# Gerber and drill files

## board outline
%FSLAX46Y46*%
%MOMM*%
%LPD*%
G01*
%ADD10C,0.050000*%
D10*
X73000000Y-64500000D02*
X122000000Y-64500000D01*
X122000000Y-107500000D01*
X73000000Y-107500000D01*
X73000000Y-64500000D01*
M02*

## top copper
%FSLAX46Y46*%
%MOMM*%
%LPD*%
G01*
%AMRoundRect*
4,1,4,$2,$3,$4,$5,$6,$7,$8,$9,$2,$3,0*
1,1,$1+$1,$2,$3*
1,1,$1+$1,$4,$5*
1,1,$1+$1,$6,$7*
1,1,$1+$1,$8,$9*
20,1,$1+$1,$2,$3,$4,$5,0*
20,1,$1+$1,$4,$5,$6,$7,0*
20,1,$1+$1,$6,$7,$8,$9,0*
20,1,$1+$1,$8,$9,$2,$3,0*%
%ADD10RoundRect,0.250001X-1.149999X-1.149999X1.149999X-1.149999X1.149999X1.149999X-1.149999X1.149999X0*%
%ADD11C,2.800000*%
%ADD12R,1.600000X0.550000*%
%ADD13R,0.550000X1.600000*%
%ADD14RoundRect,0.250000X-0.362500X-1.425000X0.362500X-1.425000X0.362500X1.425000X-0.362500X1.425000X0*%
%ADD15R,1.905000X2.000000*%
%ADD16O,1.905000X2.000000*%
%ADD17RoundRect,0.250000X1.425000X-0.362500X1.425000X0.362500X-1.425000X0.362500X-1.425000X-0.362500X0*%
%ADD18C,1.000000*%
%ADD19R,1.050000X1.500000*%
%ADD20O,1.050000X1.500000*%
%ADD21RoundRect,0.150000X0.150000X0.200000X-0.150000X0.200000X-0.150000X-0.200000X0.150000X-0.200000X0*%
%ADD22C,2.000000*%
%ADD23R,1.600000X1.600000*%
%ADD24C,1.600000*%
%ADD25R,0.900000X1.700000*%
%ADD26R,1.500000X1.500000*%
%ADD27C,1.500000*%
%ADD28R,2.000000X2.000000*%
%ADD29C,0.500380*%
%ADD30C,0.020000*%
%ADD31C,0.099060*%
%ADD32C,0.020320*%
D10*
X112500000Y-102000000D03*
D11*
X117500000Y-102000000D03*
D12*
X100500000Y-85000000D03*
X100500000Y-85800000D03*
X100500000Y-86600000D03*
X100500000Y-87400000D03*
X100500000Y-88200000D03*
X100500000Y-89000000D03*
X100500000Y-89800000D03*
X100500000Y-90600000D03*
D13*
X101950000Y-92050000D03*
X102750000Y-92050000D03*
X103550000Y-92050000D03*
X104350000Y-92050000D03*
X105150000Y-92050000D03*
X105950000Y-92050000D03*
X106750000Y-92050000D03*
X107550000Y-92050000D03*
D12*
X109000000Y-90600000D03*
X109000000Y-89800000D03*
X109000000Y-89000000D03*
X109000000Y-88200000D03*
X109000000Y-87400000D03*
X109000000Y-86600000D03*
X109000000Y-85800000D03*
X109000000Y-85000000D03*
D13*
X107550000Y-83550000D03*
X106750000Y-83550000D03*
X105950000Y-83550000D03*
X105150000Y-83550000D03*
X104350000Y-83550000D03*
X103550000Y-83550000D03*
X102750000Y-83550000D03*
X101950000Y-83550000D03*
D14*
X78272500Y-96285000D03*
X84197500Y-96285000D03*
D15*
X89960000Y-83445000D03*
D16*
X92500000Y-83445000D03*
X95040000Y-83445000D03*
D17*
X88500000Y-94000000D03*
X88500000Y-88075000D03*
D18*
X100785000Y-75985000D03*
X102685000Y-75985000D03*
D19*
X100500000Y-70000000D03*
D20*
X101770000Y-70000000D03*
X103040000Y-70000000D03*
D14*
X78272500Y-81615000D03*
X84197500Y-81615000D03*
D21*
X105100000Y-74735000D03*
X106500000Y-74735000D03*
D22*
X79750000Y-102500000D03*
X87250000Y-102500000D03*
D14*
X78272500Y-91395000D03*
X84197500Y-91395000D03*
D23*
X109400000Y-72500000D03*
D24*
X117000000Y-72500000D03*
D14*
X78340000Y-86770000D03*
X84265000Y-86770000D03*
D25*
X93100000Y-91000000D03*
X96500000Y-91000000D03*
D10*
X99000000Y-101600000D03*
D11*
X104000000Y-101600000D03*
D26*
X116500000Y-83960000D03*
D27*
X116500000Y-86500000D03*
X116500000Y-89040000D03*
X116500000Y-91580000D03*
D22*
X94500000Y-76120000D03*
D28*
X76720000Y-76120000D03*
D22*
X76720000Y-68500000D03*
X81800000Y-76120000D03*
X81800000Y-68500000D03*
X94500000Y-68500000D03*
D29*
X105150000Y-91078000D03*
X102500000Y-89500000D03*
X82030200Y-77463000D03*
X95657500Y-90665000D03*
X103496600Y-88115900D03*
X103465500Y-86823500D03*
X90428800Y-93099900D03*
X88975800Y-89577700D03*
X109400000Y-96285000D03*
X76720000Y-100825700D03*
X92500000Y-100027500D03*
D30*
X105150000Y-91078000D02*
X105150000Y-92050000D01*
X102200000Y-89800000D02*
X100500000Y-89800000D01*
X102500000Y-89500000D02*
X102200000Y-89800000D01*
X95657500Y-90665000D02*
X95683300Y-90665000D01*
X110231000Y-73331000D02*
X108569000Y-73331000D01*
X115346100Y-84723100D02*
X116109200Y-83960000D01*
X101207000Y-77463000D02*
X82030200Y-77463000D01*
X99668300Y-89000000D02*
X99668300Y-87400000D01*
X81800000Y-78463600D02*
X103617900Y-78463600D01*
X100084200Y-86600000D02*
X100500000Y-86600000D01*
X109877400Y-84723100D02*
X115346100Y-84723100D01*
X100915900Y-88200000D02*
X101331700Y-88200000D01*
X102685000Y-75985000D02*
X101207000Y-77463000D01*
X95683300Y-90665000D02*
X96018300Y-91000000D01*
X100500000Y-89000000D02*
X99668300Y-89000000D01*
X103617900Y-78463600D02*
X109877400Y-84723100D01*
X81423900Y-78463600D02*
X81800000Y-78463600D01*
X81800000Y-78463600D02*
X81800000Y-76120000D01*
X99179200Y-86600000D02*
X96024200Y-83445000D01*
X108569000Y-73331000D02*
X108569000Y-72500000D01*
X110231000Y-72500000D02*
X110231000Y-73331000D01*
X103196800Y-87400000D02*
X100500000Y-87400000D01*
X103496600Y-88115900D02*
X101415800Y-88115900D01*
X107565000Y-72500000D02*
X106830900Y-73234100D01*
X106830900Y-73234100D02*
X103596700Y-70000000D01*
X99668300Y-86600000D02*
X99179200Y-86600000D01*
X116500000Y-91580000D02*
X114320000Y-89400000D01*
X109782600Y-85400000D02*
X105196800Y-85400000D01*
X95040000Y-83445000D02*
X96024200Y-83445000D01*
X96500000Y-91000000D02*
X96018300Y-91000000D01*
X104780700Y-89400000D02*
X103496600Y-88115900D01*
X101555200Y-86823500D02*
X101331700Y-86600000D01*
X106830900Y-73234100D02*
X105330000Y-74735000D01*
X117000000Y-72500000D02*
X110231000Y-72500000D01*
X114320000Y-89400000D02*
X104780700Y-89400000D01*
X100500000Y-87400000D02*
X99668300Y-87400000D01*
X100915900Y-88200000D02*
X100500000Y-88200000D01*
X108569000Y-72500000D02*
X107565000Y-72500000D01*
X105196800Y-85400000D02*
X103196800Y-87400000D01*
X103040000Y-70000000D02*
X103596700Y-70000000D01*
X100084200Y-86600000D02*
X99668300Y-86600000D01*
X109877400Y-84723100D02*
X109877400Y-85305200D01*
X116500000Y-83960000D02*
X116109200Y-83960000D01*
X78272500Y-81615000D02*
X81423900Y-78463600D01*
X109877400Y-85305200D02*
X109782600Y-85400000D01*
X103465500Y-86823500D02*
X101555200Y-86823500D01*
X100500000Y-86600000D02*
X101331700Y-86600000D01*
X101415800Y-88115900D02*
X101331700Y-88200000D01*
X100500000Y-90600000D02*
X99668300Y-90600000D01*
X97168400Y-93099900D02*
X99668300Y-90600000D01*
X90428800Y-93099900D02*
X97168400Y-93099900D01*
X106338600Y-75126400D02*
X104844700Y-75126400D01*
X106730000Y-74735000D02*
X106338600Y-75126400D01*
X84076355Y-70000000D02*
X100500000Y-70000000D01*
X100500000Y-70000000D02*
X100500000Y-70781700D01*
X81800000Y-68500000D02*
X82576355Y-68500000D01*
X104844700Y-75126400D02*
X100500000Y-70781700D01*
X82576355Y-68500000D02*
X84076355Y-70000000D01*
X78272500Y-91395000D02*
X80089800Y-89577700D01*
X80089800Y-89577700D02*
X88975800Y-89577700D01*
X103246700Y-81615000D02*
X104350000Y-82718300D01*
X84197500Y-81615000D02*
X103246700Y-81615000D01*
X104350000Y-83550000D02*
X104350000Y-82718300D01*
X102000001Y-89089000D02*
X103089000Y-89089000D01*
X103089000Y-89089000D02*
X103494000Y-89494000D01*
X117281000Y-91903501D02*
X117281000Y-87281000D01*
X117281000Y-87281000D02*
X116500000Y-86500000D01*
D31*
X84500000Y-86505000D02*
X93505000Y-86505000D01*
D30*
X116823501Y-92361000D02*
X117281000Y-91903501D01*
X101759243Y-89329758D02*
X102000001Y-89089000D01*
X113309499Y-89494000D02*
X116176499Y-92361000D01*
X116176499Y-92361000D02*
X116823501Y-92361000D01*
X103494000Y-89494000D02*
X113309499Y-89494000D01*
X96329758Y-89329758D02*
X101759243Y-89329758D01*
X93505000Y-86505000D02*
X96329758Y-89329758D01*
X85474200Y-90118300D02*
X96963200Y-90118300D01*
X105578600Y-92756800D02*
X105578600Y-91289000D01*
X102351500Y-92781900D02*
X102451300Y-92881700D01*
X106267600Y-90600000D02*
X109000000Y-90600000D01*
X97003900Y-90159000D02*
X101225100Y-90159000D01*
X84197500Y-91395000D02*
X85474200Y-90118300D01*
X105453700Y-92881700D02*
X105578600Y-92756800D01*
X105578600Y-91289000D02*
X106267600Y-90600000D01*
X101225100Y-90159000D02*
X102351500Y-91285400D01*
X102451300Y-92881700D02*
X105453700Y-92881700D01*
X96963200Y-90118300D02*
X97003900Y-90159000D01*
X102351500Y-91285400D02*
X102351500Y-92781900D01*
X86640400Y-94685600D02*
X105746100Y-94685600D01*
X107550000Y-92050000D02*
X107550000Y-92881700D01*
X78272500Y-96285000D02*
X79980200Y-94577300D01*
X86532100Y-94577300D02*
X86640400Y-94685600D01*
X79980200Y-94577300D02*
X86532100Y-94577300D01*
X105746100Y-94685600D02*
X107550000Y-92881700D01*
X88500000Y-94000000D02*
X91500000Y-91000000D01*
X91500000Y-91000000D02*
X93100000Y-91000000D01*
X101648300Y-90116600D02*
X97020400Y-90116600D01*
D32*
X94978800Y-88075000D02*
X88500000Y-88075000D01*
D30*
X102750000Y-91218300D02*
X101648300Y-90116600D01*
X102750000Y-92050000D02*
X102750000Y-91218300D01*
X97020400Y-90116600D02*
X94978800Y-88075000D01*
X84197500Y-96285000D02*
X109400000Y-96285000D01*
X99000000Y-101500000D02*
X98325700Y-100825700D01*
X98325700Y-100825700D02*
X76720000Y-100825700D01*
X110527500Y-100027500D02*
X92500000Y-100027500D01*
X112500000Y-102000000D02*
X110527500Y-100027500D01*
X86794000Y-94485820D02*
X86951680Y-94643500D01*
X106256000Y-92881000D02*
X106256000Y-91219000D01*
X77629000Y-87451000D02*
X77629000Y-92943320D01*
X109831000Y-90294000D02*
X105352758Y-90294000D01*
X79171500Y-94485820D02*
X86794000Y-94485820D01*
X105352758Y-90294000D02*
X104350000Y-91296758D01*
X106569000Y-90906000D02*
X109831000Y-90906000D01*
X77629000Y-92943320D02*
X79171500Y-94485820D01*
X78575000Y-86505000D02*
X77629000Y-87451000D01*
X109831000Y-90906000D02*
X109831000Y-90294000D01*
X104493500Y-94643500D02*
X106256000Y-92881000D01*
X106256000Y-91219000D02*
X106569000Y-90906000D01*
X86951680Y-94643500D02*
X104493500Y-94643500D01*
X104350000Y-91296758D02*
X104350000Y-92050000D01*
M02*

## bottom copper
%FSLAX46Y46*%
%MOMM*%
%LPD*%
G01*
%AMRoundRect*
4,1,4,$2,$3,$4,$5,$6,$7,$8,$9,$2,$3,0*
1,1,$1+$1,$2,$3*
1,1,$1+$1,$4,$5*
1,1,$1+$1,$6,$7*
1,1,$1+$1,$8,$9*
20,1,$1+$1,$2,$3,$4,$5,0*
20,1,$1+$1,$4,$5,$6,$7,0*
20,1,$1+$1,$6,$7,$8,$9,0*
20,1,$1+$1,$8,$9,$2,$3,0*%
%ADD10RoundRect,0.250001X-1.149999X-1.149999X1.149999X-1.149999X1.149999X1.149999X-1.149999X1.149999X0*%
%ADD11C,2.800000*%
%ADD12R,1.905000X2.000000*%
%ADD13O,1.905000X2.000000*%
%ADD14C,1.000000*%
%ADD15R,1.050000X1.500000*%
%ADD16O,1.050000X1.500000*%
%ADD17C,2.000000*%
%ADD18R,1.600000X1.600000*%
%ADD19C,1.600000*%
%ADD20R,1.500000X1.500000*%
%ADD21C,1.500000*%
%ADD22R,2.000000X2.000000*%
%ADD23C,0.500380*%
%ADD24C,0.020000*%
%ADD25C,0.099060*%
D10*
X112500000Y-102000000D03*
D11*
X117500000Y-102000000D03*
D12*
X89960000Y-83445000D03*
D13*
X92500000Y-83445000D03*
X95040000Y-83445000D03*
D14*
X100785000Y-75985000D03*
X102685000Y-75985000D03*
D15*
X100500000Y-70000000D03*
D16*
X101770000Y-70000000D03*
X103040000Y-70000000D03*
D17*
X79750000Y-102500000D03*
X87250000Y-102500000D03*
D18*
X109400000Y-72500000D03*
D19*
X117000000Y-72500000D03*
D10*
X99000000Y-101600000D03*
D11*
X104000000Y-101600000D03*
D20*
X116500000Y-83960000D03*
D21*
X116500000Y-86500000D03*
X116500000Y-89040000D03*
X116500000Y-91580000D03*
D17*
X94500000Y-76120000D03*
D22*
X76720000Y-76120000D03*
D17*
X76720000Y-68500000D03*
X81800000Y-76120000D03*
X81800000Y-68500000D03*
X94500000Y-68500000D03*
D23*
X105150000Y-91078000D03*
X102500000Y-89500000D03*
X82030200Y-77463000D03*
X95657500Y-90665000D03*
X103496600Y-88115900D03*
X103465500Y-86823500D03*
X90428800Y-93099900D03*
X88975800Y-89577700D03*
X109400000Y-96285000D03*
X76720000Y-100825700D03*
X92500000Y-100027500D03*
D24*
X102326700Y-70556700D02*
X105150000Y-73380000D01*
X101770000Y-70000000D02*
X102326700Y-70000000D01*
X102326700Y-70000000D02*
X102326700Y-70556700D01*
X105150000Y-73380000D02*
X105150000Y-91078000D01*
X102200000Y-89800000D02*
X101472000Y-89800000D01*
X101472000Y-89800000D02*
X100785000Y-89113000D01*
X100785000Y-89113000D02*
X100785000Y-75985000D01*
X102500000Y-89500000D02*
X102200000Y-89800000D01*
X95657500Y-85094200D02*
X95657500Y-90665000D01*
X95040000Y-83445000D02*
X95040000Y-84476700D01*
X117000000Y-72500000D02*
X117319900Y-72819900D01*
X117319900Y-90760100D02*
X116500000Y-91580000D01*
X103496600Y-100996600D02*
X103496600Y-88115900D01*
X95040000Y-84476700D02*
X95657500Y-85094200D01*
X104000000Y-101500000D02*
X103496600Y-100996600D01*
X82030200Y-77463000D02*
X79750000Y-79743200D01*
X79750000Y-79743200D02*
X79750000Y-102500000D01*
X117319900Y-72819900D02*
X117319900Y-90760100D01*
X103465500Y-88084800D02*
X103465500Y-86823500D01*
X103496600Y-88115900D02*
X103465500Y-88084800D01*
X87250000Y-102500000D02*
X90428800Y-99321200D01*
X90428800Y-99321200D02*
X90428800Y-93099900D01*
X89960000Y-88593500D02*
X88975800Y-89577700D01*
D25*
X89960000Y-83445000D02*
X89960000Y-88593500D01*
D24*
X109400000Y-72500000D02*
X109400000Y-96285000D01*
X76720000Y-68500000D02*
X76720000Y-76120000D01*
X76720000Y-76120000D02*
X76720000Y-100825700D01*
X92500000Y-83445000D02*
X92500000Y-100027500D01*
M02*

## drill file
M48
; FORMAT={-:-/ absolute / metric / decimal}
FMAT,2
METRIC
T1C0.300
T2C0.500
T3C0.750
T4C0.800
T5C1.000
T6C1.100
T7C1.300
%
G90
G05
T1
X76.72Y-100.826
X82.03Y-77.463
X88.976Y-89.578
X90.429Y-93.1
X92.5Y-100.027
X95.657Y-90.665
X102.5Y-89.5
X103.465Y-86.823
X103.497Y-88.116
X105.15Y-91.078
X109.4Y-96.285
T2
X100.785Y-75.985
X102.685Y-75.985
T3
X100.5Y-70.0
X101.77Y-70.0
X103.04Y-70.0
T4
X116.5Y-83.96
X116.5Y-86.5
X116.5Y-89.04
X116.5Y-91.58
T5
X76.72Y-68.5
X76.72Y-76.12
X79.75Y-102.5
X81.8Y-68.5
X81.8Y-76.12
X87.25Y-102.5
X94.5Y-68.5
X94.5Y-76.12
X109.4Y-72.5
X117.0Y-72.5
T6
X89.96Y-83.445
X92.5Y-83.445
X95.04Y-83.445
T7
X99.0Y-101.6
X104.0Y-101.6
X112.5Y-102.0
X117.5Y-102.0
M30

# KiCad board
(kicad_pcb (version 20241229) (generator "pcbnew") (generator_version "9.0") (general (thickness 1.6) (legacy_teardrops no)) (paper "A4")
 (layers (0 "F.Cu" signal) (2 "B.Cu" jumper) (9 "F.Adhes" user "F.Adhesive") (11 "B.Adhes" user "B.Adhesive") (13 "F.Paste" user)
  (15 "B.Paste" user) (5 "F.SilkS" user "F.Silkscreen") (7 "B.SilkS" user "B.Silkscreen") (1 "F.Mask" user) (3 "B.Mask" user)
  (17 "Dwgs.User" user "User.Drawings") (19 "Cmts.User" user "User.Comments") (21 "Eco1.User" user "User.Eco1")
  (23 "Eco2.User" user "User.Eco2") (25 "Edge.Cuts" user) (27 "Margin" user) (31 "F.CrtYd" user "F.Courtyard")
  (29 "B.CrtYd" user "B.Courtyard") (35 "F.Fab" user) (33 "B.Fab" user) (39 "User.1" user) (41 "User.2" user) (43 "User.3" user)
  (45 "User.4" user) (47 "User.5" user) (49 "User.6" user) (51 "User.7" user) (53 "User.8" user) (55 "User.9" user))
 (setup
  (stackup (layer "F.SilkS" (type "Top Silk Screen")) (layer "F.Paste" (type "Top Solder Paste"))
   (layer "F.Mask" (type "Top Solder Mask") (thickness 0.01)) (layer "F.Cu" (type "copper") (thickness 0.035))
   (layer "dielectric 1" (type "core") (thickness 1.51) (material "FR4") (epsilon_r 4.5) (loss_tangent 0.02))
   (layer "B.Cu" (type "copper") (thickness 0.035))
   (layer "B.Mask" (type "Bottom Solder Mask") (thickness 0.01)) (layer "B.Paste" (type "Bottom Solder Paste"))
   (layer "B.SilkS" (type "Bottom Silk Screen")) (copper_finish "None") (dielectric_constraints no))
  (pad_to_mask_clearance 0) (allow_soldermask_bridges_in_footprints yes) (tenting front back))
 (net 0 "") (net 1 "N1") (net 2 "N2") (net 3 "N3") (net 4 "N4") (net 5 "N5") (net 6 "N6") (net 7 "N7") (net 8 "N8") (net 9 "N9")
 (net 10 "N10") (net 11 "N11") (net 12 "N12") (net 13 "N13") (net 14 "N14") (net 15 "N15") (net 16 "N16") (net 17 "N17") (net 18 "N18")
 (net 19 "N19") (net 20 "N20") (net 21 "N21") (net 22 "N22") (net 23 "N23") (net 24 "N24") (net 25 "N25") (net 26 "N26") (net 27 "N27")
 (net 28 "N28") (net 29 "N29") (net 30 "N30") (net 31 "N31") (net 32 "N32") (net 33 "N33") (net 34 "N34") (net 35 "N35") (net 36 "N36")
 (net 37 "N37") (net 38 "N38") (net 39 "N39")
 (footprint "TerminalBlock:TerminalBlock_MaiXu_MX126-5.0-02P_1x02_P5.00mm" (layer "F.Cu") (at 112.5 102)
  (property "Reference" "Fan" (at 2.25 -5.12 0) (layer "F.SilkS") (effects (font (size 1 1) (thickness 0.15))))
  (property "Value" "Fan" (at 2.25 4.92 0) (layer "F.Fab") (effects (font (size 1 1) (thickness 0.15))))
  (pad "1" thru_hole roundrect (at 0 0) (size 2.8 2.8) (drill 1.3) (layers "*.Cu" "*.Mask") (remove_unused_layers no)
   (roundrect_rratio 0.089286) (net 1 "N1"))
  (pad "2" thru_hole circle (at 5 0) (size 2.8 2.8) (drill 1.3) (layers "*.Cu" "*.Mask") (remove_unused_layers no) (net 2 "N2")))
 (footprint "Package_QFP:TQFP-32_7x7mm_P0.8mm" (layer "F.Cu") (at 104.75 87.8)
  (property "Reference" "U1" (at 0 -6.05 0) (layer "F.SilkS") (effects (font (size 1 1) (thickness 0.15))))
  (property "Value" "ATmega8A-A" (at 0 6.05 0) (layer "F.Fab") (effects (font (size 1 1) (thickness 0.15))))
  (pad "1" smd rect (at -4.25 -2.8) (size 1.6 0.55) (layers "F.Cu" "F.Mask" "F.Paste") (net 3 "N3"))
  (pad "2" smd rect (at -4.25 -2) (size 1.6 0.55) (layers "F.Cu" "F.Mask" "F.Paste") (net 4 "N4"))
  (pad "3" smd rect (at -4.25 -1.2) (size 1.6 0.55) (layers "F.Cu" "F.Mask" "F.Paste") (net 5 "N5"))
  (pad "4" smd rect (at -4.25 -0.4) (size 1.6 0.55) (layers "F.Cu" "F.Mask" "F.Paste") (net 5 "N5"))
  (pad "5" smd rect (at -4.25 0.4) (size 1.6 0.55) (layers "F.Cu" "F.Mask" "F.Paste") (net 5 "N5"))
  (pad "6" smd rect (at -4.25 1.2) (size 1.6 0.55) (layers "F.Cu" "F.Mask" "F.Paste") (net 5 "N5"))
  (pad "7" smd rect (at -4.25 2) (size 1.6 0.55) (layers "F.Cu" "F.Mask" "F.Paste") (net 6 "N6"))
  (pad "8" smd rect (at -4.25 2.8) (size 1.6 0.55) (layers "F.Cu" "F.Mask" "F.Paste") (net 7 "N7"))
  (pad "9" smd rect (at -2.8 4.25 90) (size 1.6 0.55) (layers "F.Cu" "F.Mask" "F.Paste") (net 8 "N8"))
  (pad "10" smd rect (at -2 4.25 90) (size 1.6 0.55) (layers "F.Cu" "F.Mask" "F.Paste") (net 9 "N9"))
  (pad "11" smd rect (at -1.2 4.25 90) (size 1.6 0.55) (layers "F.Cu" "F.Mask" "F.Paste") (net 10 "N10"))
  (pad "12" smd rect (at -0.4 4.25 90) (size 1.6 0.55) (layers "F.Cu" "F.Mask" "F.Paste") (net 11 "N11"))
  (pad "13" smd rect (at 0.4 4.25 90) (size 1.6 0.55) (layers "F.Cu" "F.Mask" "F.Paste") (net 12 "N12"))
  (pad "14" smd rect (at 1.2 4.25 90) (size 1.6 0.55) (layers "F.Cu" "F.Mask" "F.Paste") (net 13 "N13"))
  (pad "15" smd rect (at 2 4.25 90) (size 1.6 0.55) (layers "F.Cu" "F.Mask" "F.Paste") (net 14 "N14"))
  (pad "16" smd rect (at 2.8 4.25 90) (size 1.6 0.55) (layers "F.Cu" "F.Mask" "F.Paste") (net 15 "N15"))
  (pad "17" smd rect (at 4.25 2.8) (size 1.6 0.55) (layers "F.Cu" "F.Mask" "F.Paste") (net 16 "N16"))
  (pad "18" smd rect (at 4.25 2) (size 1.6 0.55) (layers "F.Cu" "F.Mask" "F.Paste") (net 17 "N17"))
  (pad "19" smd rect (at 4.25 1.2) (size 1.6 0.55) (layers "F.Cu" "F.Mask" "F.Paste") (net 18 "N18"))
  (pad "20" smd rect (at 4.25 0.4) (size 1.6 0.55) (layers "F.Cu" "F.Mask" "F.Paste") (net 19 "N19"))
  (pad "21" smd rect (at 4.25 -0.4) (size 1.6 0.55) (layers "F.Cu" "F.Mask" "F.Paste") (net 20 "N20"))
  (pad "22" smd rect (at 4.25 -1.2) (size 1.6 0.55) (layers "F.Cu" "F.Mask" "F.Paste") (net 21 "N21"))
  (pad "23" smd rect (at 4.25 -2) (size 1.6 0.55) (layers "F.Cu" "F.Mask" "F.Paste") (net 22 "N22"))
  (pad "24" smd rect (at 4.25 -2.8) (size 1.6 0.55) (layers "F.Cu" "F.Mask" "F.Paste") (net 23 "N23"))
  (pad "25" smd rect (at 2.8 -4.25 90) (size 1.6 0.55) (layers "F.Cu" "F.Mask" "F.Paste") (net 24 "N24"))
  (pad "26" smd rect (at 2 -4.25 90) (size 1.6 0.55) (layers "F.Cu" "F.Mask" "F.Paste") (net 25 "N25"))
  (pad "27" smd rect (at 1.2 -4.25 90) (size 1.6 0.55) (layers "F.Cu" "F.Mask" "F.Paste") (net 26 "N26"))
  (pad "28" smd rect (at 0.4 -4.25 90) (size 1.6 0.55) (layers "F.Cu" "F.Mask" "F.Paste") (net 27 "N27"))
  (pad "29" smd rect (at -0.4 -4.25 90) (size 1.6 0.55) (layers "F.Cu" "F.Mask" "F.Paste") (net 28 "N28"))
  (pad "30" smd rect (at -1.2 -4.25 90) (size 1.6 0.55) (layers "F.Cu" "F.Mask" "F.Paste") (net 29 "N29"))
  (pad "31" smd rect (at -2 -4.25 90) (size 1.6 0.55) (layers "F.Cu" "F.Mask" "F.Paste") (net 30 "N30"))
  (pad "32" smd rect (at -2.8 -4.25 90) (size 1.6 0.55) (layers "F.Cu" "F.Mask" "F.Paste") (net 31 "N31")))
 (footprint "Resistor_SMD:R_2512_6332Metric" (layer "F.Cu") (at 81.235 96.285)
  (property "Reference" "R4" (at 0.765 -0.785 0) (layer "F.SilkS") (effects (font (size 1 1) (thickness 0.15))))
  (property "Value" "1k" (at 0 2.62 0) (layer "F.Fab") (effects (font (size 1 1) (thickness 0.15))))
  (pad "1" smd roundrect (at -2.9625 0) (size 1.225 3.35) (layers "F.Cu" "F.Mask" "F.Paste") (roundrect_rratio 0.204082) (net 15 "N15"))
  (pad "2" smd roundrect (at 2.9625 0) (size 1.225 3.35) (layers "F.Cu" "F.Mask" "F.Paste") (roundrect_rratio 0.204082) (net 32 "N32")))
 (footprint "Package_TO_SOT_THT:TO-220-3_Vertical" (layer "F.Cu") (at 89.96 83.445)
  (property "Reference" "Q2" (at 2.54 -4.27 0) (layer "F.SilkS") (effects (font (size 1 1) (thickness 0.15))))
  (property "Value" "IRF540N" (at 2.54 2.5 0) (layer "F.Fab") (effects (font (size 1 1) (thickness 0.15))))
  (pad "1" thru_hole rect (at 0 0) (size 1.905 2) (drill 1.1) (layers "*.Cu" "*.Mask") (remove_unused_layers no) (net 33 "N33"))
  (pad "2" thru_hole oval (at 2.54 0) (size 1.905 2) (drill 1.1) (layers "*.Cu" "*.Mask") (remove_unused_layers no) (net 1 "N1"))
  (pad "3" thru_hole oval (at 5.08 0) (size 1.905 2) (drill 1.1) (layers "*.Cu" "*.Mask") (remove_unused_layers no) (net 5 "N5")))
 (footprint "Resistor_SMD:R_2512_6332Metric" (layer "F.Cu") (at 88.5 91.0375 90)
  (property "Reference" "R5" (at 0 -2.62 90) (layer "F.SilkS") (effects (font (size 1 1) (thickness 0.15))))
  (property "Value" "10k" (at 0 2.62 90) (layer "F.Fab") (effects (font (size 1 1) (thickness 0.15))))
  (pad "1" smd roundrect (at -2.9625 0 90) (size 1.225 3.35) (layers "F.Cu" "F.Mask" "F.Paste") (roundrect_rratio 0.204082) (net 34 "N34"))
  (pad "2" smd roundrect (at 2.9625 0 90) (size 1.225 3.35) (layers "F.Cu" "F.Mask" "F.Paste") (roundrect_rratio 0.204082) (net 9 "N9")))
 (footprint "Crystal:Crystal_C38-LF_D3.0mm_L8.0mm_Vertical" (layer "F.Cu") (at 100.785 75.985)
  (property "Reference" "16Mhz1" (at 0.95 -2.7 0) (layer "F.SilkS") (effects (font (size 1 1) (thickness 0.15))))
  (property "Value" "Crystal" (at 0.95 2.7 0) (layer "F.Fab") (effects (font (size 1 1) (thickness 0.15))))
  (pad "1" thru_hole circle (at 0 0) (size 1 1) (drill 0.5) (layers "*.Cu" "*.Mask") (remove_unused_layers no) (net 6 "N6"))
  (pad "2" thru_hole circle (at 1.9 0) (size 1 1) (drill 0.5) (layers "*.Cu" "*.Mask") (remove_unused_layers no) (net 5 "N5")))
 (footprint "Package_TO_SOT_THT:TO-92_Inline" (layer "F.Cu") (at 100.5 70)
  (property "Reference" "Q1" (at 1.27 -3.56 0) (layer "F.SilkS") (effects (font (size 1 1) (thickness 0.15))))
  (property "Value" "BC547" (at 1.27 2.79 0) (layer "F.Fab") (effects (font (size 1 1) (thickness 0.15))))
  (pad "1" thru_hole rect (at 0 0) (size 1.05 1.5) (drill 0.75) (layers "*.Cu" "*.Mask") (remove_unused_layers no) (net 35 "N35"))
  (pad "2" thru_hole oval (at 1.27 0) (size 1.05 1.5) (drill 0.75) (layers "*.Cu" "*.Mask") (remove_unused_layers no) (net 12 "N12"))
  (pad "3" thru_hole oval (at 2.54 0) (size 1.05 1.5) (drill 0.75) (layers "*.Cu" "*.Mask") (remove_unused_layers no) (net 5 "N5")))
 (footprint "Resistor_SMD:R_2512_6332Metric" (layer "F.Cu") (at 81.235 81.615)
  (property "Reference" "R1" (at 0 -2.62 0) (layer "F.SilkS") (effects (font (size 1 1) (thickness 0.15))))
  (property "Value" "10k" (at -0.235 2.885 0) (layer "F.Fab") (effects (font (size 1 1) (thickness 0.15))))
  (pad "1" smd roundrect (at -2.9625 0) (size 1.225 3.35) (layers "F.Cu" "F.Mask" "F.Paste") (roundrect_rratio 0.204082) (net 5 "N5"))
  (pad "2" smd roundrect (at 2.9625 0) (size 1.225 3.35) (layers "F.Cu" "F.Mask" "F.Paste") (roundrect_rratio 0.204082) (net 28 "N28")))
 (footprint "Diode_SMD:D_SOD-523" (layer "F.Cu") (at 105.8 74.735)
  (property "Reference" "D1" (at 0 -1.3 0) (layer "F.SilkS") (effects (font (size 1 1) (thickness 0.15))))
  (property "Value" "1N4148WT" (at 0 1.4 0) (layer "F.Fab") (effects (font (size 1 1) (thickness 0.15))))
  (pad "1" smd roundrect (at -0.7 0 180) (size 0.6 0.7) (layers "F.Cu" "F.Mask" "F.Paste") (roundrect_rratio 0.25) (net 5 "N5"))
  (pad "2" smd roundrect (at 0.7 0 180) (size 0.6 0.7) (layers "F.Cu" "F.Mask" "F.Paste") (roundrect_rratio 0.25) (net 35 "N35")))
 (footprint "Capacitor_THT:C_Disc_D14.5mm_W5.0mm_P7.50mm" (layer "F.Cu") (at 79.75 102.5)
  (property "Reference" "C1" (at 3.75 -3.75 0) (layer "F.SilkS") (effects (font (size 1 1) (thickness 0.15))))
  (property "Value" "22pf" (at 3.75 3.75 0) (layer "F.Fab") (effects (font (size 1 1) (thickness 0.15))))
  (pad "1" thru_hole circle (at 0 0) (size 2 2) (drill 1) (layers "*.Cu" "*.Mask") (remove_unused_layers no) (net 5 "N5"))
  (pad "2" thru_hole circle (at 7.5 0) (size 2 2) (drill 1) (layers "*.Cu" "*.Mask") (remove_unused_layers no) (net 7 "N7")))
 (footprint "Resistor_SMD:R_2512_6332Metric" (layer "F.Cu") (at 81.235 91.395)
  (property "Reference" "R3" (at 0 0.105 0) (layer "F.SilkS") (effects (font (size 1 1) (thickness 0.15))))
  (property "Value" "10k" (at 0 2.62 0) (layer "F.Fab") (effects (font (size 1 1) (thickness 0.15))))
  (pad "1" smd roundrect (at -2.9625 0) (size 1.225 3.35) (layers "F.Cu" "F.Mask" "F.Paste") (roundrect_rratio 0.204082) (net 33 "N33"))
  (pad "2" smd roundrect (at 2.9625 0) (size 1.225 3.35) (layers "F.Cu" "F.Mask" "F.Paste") (roundrect_rratio 0.204082) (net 16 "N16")))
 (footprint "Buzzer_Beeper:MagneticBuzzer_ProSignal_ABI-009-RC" (layer "F.Cu") (at 109.4 72.5)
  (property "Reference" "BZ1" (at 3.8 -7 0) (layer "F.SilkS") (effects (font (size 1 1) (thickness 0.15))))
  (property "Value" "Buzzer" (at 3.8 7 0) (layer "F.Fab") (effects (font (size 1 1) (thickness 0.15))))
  (pad "1" thru_hole rect (at 0 0) (size 1.6 1.6) (drill 1) (layers "*.Cu" "*.Mask") (remove_unused_layers no) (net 32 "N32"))
  (pad "2" thru_hole circle (at 7.6 0) (size 1.6 1.6) (drill 1) (layers "*.Cu" "*.Mask") (remove_unused_layers no) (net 5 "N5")))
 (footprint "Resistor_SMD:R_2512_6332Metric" (layer "F.Cu") (at 81.3025 86.77)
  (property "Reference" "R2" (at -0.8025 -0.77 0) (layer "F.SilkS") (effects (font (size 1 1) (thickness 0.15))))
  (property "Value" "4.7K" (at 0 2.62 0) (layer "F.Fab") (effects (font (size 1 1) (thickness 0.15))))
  (pad "1" smd roundrect (at -2.9625 0) (size 1.225 3.35) (layers "F.Cu" "F.Mask" "F.Paste") (roundrect_rratio 0.204082) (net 11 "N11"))
  (pad "2" smd roundrect (at 2.9625 0) (size 1.225 3.35) (layers "F.Cu" "F.Mask" "F.Paste") (roundrect_rratio 0.204082) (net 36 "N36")))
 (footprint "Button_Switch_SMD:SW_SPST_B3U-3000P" (layer "F.Cu") (at 94.8 91)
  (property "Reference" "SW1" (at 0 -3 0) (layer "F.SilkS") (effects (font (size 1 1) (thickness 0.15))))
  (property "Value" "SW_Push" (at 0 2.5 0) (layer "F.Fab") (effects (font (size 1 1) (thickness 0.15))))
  (pad "1" smd rect (at -1.7 0) (size 0.9 1.7) (layers "F.Cu" "F.Mask" "F.Paste") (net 34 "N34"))
  (pad "2" smd rect (at 1.7 0) (size 0.9 1.7) (layers "F.Cu" "F.Mask" "F.Paste") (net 5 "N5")))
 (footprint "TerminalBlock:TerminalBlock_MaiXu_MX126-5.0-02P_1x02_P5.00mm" (layer "F.Cu") (at 99 101.6)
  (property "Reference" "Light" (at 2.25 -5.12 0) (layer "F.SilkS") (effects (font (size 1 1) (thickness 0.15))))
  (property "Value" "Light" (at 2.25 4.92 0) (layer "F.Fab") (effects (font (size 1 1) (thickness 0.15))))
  (pad "1" thru_hole roundrect (at 0 0) (size 2.8 2.8) (drill 1.3) (layers "*.Cu" "*.Mask") (remove_unused_layers no)
   (roundrect_rratio 0.089286) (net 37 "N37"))
  (pad "2" thru_hole circle (at 5 0) (size 2.8 2.8) (drill 1.3) (layers "*.Cu" "*.Mask") (remove_unused_layers no) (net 5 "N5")))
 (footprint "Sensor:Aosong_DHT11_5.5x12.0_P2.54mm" (layer "F.Cu") (at 116.5 83.96)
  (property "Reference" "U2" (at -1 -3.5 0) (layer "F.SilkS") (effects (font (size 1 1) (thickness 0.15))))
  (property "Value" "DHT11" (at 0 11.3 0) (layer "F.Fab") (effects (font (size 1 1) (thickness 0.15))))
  (pad "1" thru_hole rect (at 0 0) (size 1.5 1.5) (drill 0.8) (layers "*.Cu" "*.Mask") (remove_unused_layers no) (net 5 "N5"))
  (pad "2" thru_hole circle (at 0 2.54) (size 1.5 1.5) (drill 0.8) (layers "*.Cu" "*.Mask") (remove_unused_layers no) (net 36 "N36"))
  (pad "3" thru_hole circle (at 0 5.08) (size 1.5 1.5) (drill 0.8) (layers "*.Cu" "*.Mask") (remove_unused_layers no) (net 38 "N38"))
  (pad "4" thru_hole circle (at 0 7.62) (size 1.5 1.5) (drill 0.8) (layers "*.Cu" "*.Mask") (remove_unused_layers no) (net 5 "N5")))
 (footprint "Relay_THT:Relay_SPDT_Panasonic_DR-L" (layer "F.Cu") (at 76.72 76.12)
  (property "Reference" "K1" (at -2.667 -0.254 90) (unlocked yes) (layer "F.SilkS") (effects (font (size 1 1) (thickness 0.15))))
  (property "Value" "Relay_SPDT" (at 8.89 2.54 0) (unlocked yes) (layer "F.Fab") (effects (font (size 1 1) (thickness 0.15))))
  (pad "11" thru_hole circle (at 17.78 0 180) (size 2 2) (drill 1) (layers "*.Cu" "*.Mask") (remove_unused_layers no) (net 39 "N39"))
  (pad "12" thru_hole rect (at 0 0 180) (size 2 2) (drill 1) (layers "*.Cu" "*.Mask") (remove_unused_layers no) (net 37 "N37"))
  (pad "14" thru_hole circle (at 0 -7.62 180) (size 2 2) (drill 1) (layers "*.Cu" "*.Mask") (remove_unused_layers no) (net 37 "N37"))
  (pad "A1" thru_hole circle (at 5.08 0 180) (size 2 2) (drill 1) (layers "*.Cu" "*.Mask") (remove_unused_layers no) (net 5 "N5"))
  (pad "A2" thru_hole circle (at 5.08 -7.62 180) (size 2 2) (drill 1) (layers "*.Cu" "*.Mask") (remove_unused_layers no) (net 35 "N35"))
  (pad "PE" thru_hole circle (at 17.78 -7.62 180) (size 2 2) (drill 1) (layers "*.Cu" "*.Mask") (remove_unused_layers no)))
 (gr_rect (start 73 64.5) (end 122 107.5) (stroke (width 0.05) (type default)) (fill no) (layer "Edge.Cuts"))
 (segment (start 105.15 91.078) (end 105.15 92.05) (width 0.02) (layer "F.Cu") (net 12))
 (via (at 105.15 91.078) (size 0.50038) (drill 0.3) (layers "F.Cu" "B.Cu") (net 12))
 (segment (start 102.3267 70.5567) (end 105.15 73.38) (width 0.02) (layer "B.Cu") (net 12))
 (segment (start 101.77 70) (end 102.3267 70) (width 0.02) (layer "B.Cu") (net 12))
 (segment (start 102.3267 70) (end 102.3267 70.5567) (width 0.02) (layer "B.Cu") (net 12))
 (segment (start 105.15 73.38) (end 105.15 91.078) (width 0.02) (layer "B.Cu") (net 12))
 (segment (start 102.2 89.8) (end 100.5 89.8) (width 0.02) (layer "F.Cu") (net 6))
 (segment (start 102.5 89.5) (end 102.2 89.8) (width 0.02) (layer "F.Cu") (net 6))
 (via (at 102.5 89.5) (size 0.50038) (drill 0.3) (layers "F.Cu" "B.Cu") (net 6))
 (segment (start 102.2 89.8) (end 101.472 89.8) (width 0.02) (layer "B.Cu") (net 6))
 (segment (start 101.472 89.8) (end 100.785 89.113) (width 0.02) (layer "B.Cu") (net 6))
 (segment (start 100.785 89.113) (end 100.785 75.985) (width 0.02) (layer "B.Cu") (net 6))
 (segment (start 102.5 89.5) (end 102.2 89.8) (width 0.02) (layer "B.Cu") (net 6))
 (segment (start 95.6575 90.665) (end 95.6833 90.665) (width 0.02) (layer "F.Cu") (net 5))
 (segment (start 110.231 73.331) (end 108.569 73.331) (width 0.02) (layer "F.Cu") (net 5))
 (segment (start 115.3461 84.7231) (end 116.1092 83.96) (width 0.02) (layers "F.Cu" "F.Mask") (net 5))
 (segment (start 101.207 77.463) (end 82.0302 77.463) (width 0.02) (layer "F.Cu") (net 5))
 (segment (start 99.6683 89) (end 99.6683 87.4) (width 0.02) (layer "F.Cu") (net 5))
 (segment (start 81.8 78.4636) (end 103.6179 78.4636) (width 0.02) (layer "F.Cu") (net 5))
 (segment (start 100.0842 86.6) (end 100.5 86.6) (width 0.02) (layer "F.Cu") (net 5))
 (segment (start 109.8774 84.7231) (end 115.3461 84.7231) (width 0.02) (layer "F.Cu") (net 5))
 (segment (start 100.9159 88.2) (end 101.3317 88.2) (width 0.02) (layer "F.Cu") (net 5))
 (segment (start 102.685 75.985) (end 101.207 77.463) (width 0.02) (layer "F.Cu") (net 5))
 (segment (start 95.6833 90.665) (end 96.0183 91) (width 0.02) (layer "F.Cu") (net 5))
 (segment (start 100.5 89) (end 99.6683 89) (width 0.02) (layer "F.Cu") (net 5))
 (segment (start 103.6179 78.4636) (end 109.8774 84.7231) (width 0.02) (layer "F.Cu") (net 5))
 (segment (start 81.4239 78.4636) (end 81.8 78.4636) (width 0.02) (layer "F.Cu") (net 5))
 (segment (start 81.8 78.4636) (end 81.8 76.12) (width 0.02) (layer "F.Cu") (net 5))
 (segment (start 99.1792 86.6) (end 96.0242 83.445) (width 0.02) (layer "F.Cu") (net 5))
 (segment (start 108.569 73.331) (end 108.569 72.5) (width 0.02) (layer "F.Cu") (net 5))
 (segment (start 110.231 72.5) (end 110.231 73.331) (width 0.02) (layer "F.Cu") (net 5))
 (segment (start 103.1968 87.4) (end 100.5 87.4) (width 0.02) (layer "F.Cu") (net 5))
 (segment (start 103.4966 88.1159) (end 101.4158 88.1159) (width 0.02) (layer "F.Cu") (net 5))
 (segment (start 107.565 72.5) (end 106.8309 73.2341) (width 0.02) (layer "F.Cu") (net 5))
 (segment (start 106.8309 73.2341) (end 103.5967 70) (width 0.02) (layer "F.Cu") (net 5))
 (segment (start 99.6683 86.6) (end 99.1792 86.6) (width 0.02) (layer "F.Cu") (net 5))
 (segment (start 116.5 91.58) (end 114.32 89.4) (width 0.02) (layer "F.Cu") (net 5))
 (segment (start 109.7826 85.4) (end 105.1968 85.4) (width 0.02) (layer "F.Cu") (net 5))
 (segment (start 95.04 83.445) (end 96.0242 83.445) (width 0.02) (layer "F.Cu") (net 5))
 (segment (start 96.5 91) (end 96.0183 91) (width 0.02) (layer "F.Cu") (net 5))
 (segment (start 104.7807 89.4) (end 103.4966 88.1159) (width 0.02) (layer "F.Cu") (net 5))
 (segment (start 101.5552 86.8235) (end 101.3317 86.6) (width 0.02) (layer "F.Cu") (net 5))
 (segment (start 106.8309 73.2341) (end 105.33 74.735) (width 0.02) (layer "F.Cu") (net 5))
 (segment (start 117 72.5) (end 110.231 72.5) (width 0.02) (layer "F.Cu") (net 5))
 (segment (start 114.32 89.4) (end 104.7807 89.4) (width 0.02) (layer "F.Cu") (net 5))
 (segment (start 100.5 87.4) (end 99.6683 87.4) (width 0.02) (layer "F.Cu") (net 5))
 (segment (start 100.9159 88.2) (end 100.5 88.2) (width 0.02) (layer "F.Cu") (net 5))
 (segment (start 108.569 72.5) (end 107.565 72.5) (width 0.02) (layer "F.Cu") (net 5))
 (segment (start 105.1968 85.4) (end 103.1968 87.4) (width 0.02) (layer "F.Cu") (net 5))
 (segment (start 103.04 70) (end 103.5967 70) (width 0.02) (layer "F.Cu") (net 5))
 (segment (start 100.0842 86.6) (end 99.6683 86.6) (width 0.02) (layer "F.Cu") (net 5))
 (segment (start 109.8774 84.7231) (end 109.8774 85.3052) (width 0.02) (layer "F.Cu") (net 5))
 (segment (start 116.5 83.96) (end 116.1092 83.96) (width 0.02) (layer "F.Cu") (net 5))
 (segment (start 78.2725 81.615) (end 81.4239 78.4636) (width 0.02) (layer "F.Cu") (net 5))
 (segment (start 109.8774 85.3052) (end 109.7826 85.4) (width 0.02) (layer "F.Cu") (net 5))
 (segment (start 103.4655 86.8235) (end 101.5552 86.8235) (width 0.02) (layer "F.Cu") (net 5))
 (segment (start 100.5 86.6) (end 101.3317 86.6) (width 0.02) (layer "F.Cu") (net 5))
 (segment (start 101.4158 88.1159) (end 101.3317 88.2) (width 0.02) (layer "F.Cu") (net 5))
 (via (at 82.0302 77.463) (size 0.50038) (drill 0.3) (layers "F.Cu" "B.Cu") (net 5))
 (via (at 95.6575 90.665) (size 0.50038) (drill 0.3) (layers "F.Cu" "B.Cu") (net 5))
 (via (at 103.4966 88.1159) (size 0.50038) (drill 0.3) (layers "F.Cu" "B.Cu") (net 5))
 (via (at 103.4655 86.8235) (size 0.50038) (drill 0.3) (layers "F.Cu" "B.Cu") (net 5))
 (segment (start 95.6575 85.0942) (end 95.6575 90.665) (width 0.02) (layer "B.Cu") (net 5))
 (segment (start 95.04 83.445) (end 95.04 84.4767) (width 0.02) (layer "B.Cu") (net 5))
 (segment (start 117 72.5) (end 117.3199 72.8199) (width 0.02) (layer "B.Cu") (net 5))
 (segment (start 117.3199 90.7601) (end 116.5 91.58) (width 0.02) (layer "B.Cu") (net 5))
 (segment (start 103.4966 100.9966) (end 103.4966 88.1159) (width 0.02) (layer "B.Cu") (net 5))
 (segment (start 95.04 84.4767) (end 95.6575 85.0942) (width 0.02) (layer "B.Cu") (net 5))
 (segment (start 104 101.5) (end 103.4966 100.9966) (width 0.02) (layer "B.Cu") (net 5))
 (segment (start 82.0302 77.463) (end 79.75 79.7432) (width 0.02) (layer "B.Cu") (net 5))
 (segment (start 79.75 79.7432) (end 79.75 102.5) (width 0.02) (layer "B.Cu") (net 5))
 (segment (start 117.3199 72.8199) (end 117.3199 90.7601) (width 0.02) (layer "B.Cu") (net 5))
 (segment (start 103.4655 88.0848) (end 103.4655 86.8235) (width 0.02) (layer "B.Cu") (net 5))
 (segment (start 103.4966 88.1159) (end 103.4655 88.0848) (width 0.02) (layer "B.Cu") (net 5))
 (segment (start 100.5 90.6) (end 99.6683 90.6) (width 0.02) (layer "F.Cu") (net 7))
 (segment (start 97.1684 93.0999) (end 99.6683 90.6) (width 0.02) (layer "F.Cu") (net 7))
 (segment (start 90.4288 93.0999) (end 97.1684 93.0999) (width 0.02) (layer "F.Cu") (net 7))
 (via (at 90.4288 93.0999) (size 0.50038) (drill 0.3) (layers "F.Cu" "B.Cu") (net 7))
 (segment (start 87.25 102.5) (end 90.4288 99.3212) (width 0.02) (layer "B.Cu") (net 7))
 (segment (start 90.4288 99.3212) (end 90.4288 93.0999) (width 0.02) (layer "B.Cu") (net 7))
 (segment (start 106.3386 75.1264) (end 104.8447 75.1264) (width 0.02) (layer "F.Cu") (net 35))
 (segment (start 106.73 74.735) (end 106.3386 75.1264) (width 0.02) (layer "F.Cu") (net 35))
 (segment (start 84.076355 70) (end 100.5 70) (width 0.02) (layer "F.Cu") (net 35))
 (segment (start 100.5 70) (end 100.5 70.7817) (width 0.02) (layer "F.Cu") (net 35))
 (segment (start 81.8 68.5) (end 82.576355 68.5) (width 0.02) (layer "F.Cu") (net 35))
 (segment (start 104.8447 75.1264) (end 100.5 70.7817) (width 0.02) (layer "F.Cu") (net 35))
 (segment (start 82.576355 68.5) (end 84.076355 70) (width 0.02) (layer "F.Cu") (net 35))
 (segment (start 78.2725 91.395) (end 80.0898 89.5777) (width 0.02) (layer "F.Cu") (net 33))
 (segment (start 80.0898 89.5777) (end 88.9758 89.5777) (width 0.02) (layer "F.Cu") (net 33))
 (via (at 88.9758 89.5777) (size 0.50038) (drill 0.3) (layers "F.Cu" "B.Cu") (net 33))
 (segment (start 89.96 88.5935) (end 88.9758 89.5777) (width 0.02) (layer "B.Cu") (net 33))
 (segment (start 89.96 83.445) (end 89.96 88.5935) (width 0.09906) (layer "B.Cu") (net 33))
 (segment (start 103.2467 81.615) (end 104.35 82.7183) (width 0.02) (layer "F.Cu") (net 28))
 (segment (start 84.1975 81.615) (end 103.2467 81.615) (width 0.02) (layer "F.Cu") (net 28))
 (segment (start 104.35 83.55) (end 104.35 82.7183) (width 0.02) (layer "F.Cu") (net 28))
 (segment (start 102.000001 89.089) (end 103.089 89.089) (width 0.02) (layer "F.Cu") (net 36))
 (segment (start 103.089 89.089) (end 103.494 89.494) (width 0.02) (layer "F.Cu") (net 36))
 (segment (start 117.281 91.903501) (end 117.281 87.281) (width 0.02) (layer "F.Cu") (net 36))
 (segment (start 117.281 87.281) (end 116.5 86.5) (width 0.02) (layer "F.Cu") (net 36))
 (segment (start 84.5 86.505) (end 93.505 86.505) (width 0.09906) (layer "F.Cu") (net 36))
 (segment (start 116.823501 92.361) (end 117.281 91.903501) (width 0.02) (layer "F.Cu") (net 36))
 (segment (start 101.759243 89.329758) (end 102.000001 89.089) (width 0.02) (layer "F.Cu") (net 36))
 (segment (start 113.309499 89.494) (end 116.176499 92.361) (width 0.02) (layer "F.Cu") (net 36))
 (segment (start 116.176499 92.361) (end 116.823501 92.361) (width 0.02) (layer "F.Cu") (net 36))
 (segment (start 103.494 89.494) (end 113.309499 89.494) (width 0.02) (layer "F.Cu") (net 36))
 (segment (start 96.329758 89.329758) (end 101.759243 89.329758) (width 0.02) (layer "F.Cu") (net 36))
 (segment (start 93.505 86.505) (end 96.329758 89.329758) (width 0.02) (layer "F.Cu") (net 36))
 (segment (start 85.4742 90.1183) (end 96.9632 90.1183) (width 0.02) (layer "F.Cu") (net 16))
 (segment (start 105.5786 92.7568) (end 105.5786 91.289) (width 0.02) (layer "F.Cu") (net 16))
 (segment (start 102.3515 92.7819) (end 102.4513 92.8817) (width 0.02) (layer "F.Cu") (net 16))
 (segment (start 106.2676 90.6) (end 109 90.6) (width 0.02) (layer "F.Cu") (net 16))
 (segment (start 97.0039 90.159) (end 101.2251 90.159) (width 0.02) (layer "F.Cu") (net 16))
 (segment (start 84.1975 91.395) (end 85.4742 90.1183) (width 0.02) (layer "F.Cu") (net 16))
 (segment (start 105.4537 92.8817) (end 105.5786 92.7568) (width 0.02) (layer "F.Cu") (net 16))
 (segment (start 105.5786 91.289) (end 106.2676 90.6) (width 0.02) (layer "F.Cu") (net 16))
 (segment (start 101.2251 90.159) (end 102.3515 91.2854) (width 0.02) (layer "F.Cu") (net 16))
 (segment (start 102.4513 92.8817) (end 105.4537 92.8817) (width 0.02) (layer "F.Cu") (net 16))
 (segment (start 96.9632 90.1183) (end 97.0039 90.159) (width 0.02) (layer "F.Cu") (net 16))
 (segment (start 102.3515 91.2854) (end 102.3515 92.7819) (width 0.02) (layer "F.Cu") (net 16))
 (segment (start 86.6404 94.6856) (end 105.7461 94.6856) (width 0.02) (layer "F.Cu") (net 15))
 (segment (start 107.55 92.05) (end 107.55 92.8817) (width 0.02) (layer "F.Cu") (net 15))
 (segment (start 78.2725 96.285) (end 79.9802 94.5773) (width 0.02) (layer "F.Cu") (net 15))
 (segment (start 86.5321 94.5773) (end 86.6404 94.6856) (width 0.02) (layer "F.Cu") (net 15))
 (segment (start 79.9802 94.5773) (end 86.5321 94.5773) (width 0.02) (layer "F.Cu") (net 15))
 (segment (start 105.7461 94.6856) (end 107.55 92.8817) (width 0.02) (layer "F.Cu") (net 15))
 (segment (start 88.5 94) (end 91.5 91) (width 0.02) (layer "F.Cu") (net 34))
 (segment (start 91.5 91) (end 93.1 91) (width 0.02) (layer "F.Cu") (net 34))
 (segment (start 101.6483 90.1166) (end 97.0204 90.1166) (width 0.02) (layer "F.Cu") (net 9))
 (segment (start 94.9788 88.075) (end 88.5 88.075) (width 0.02032) (layer "F.Cu") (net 9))
 (segment (start 102.75 91.2183) (end 101.6483 90.1166) (width 0.02) (layer "F.Cu") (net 9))
 (segment (start 102.75 92.05) (end 102.75 91.2183) (width 0.02) (layer "F.Cu") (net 9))
 (segment (start 97.0204 90.1166) (end 94.9788 88.075) (width 0.02) (layer "F.Cu") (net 9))
 (segment (start 84.1975 96.285) (end 109.4 96.285) (width 0.02) (layer "F.Cu") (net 32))
 (via (at 109.4 96.285) (size 0.50038) (drill 0.3) (layers "F.Cu" "B.Cu") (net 32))
 (segment (start 109.4 72.5) (end 109.4 96.285) (width 0.02) (layer "B.Cu") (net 32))
 (segment (start 99 101.5) (end 98.3257 100.8257) (width 0.02) (layer "F.Cu") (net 37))
 (segment (start 98.3257 100.8257) (end 76.72 100.8257) (width 0.02) (layer "F.Cu") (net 37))
 (via (at 76.72 100.8257) (size 0.50038) (drill 0.3) (layers "F.Cu" "B.Cu") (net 37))
 (segment (start 76.72 68.5) (end 76.72 76.12) (width 0.02) (layer "B.Cu") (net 37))
 (segment (start 76.72 76.12) (end 76.72 100.8257) (width 0.02) (layer "B.Cu") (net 37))
 (segment (start 110.5275 100.0275) (end 92.5 100.0275) (width 0.02) (layer "F.Cu") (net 1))
 (segment (start 112.5 102) (end 110.5275 100.0275) (width 0.02) (layer "F.Cu") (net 1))
 (via (at 92.5 100.0275) (size 0.50038) (drill 0.3) (layers "F.Cu" "B.Cu") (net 1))
 (segment (start 92.5 83.445) (end 92.5 100.0275) (width 0.02) (layer "B.Cu") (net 1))
 (segment (start 86.794 94.48582) (end 86.95168 94.6435) (width 0.02) (layer "F.Cu") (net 11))
 (segment (start 106.256 92.881) (end 106.256 91.219) (width 0.02) (layer "F.Cu") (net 11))
 (segment (start 77.629 87.451) (end 77.629 92.94332) (width 0.02) (layer "F.Cu") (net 11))
 (segment (start 109.831 90.294) (end 105.352758 90.294) (width 0.02) (layer "F.Cu") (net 11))
 (segment (start 79.1715 94.48582) (end 86.794 94.48582) (width 0.02) (layer "F.Cu") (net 11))
 (segment (start 105.352758 90.294) (end 104.35 91.296758) (width 0.02) (layer "F.Cu") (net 11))
 (segment (start 106.569 90.906) (end 109.831 90.906) (width 0.02) (layer "F.Cu") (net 11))
 (segment (start 77.629 92.94332) (end 79.1715 94.48582) (width 0.02) (layer "F.Cu") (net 11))
 (segment (start 78.575 86.505) (end 77.629 87.451) (width 0.02) (layer "F.Cu") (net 11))
 (segment (start 109.831 90.906) (end 109.831 90.294) (width 0.02) (layer "F.Cu") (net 11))
 (segment (start 104.4935 94.6435) (end 106.256 92.881) (width 0.02) (layer "F.Cu") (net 11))
 (segment (start 106.256 91.219) (end 106.569 90.906) (width 0.02) (layer "F.Cu") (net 11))
 (segment (start 86.95168 94.6435) (end 104.4935 94.6435) (width 0.02) (layer "F.Cu") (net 11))
 (segment (start 104.35 91.296758) (end 104.35 92.05) (width 0.02) (layer "F.Cu") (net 11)))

